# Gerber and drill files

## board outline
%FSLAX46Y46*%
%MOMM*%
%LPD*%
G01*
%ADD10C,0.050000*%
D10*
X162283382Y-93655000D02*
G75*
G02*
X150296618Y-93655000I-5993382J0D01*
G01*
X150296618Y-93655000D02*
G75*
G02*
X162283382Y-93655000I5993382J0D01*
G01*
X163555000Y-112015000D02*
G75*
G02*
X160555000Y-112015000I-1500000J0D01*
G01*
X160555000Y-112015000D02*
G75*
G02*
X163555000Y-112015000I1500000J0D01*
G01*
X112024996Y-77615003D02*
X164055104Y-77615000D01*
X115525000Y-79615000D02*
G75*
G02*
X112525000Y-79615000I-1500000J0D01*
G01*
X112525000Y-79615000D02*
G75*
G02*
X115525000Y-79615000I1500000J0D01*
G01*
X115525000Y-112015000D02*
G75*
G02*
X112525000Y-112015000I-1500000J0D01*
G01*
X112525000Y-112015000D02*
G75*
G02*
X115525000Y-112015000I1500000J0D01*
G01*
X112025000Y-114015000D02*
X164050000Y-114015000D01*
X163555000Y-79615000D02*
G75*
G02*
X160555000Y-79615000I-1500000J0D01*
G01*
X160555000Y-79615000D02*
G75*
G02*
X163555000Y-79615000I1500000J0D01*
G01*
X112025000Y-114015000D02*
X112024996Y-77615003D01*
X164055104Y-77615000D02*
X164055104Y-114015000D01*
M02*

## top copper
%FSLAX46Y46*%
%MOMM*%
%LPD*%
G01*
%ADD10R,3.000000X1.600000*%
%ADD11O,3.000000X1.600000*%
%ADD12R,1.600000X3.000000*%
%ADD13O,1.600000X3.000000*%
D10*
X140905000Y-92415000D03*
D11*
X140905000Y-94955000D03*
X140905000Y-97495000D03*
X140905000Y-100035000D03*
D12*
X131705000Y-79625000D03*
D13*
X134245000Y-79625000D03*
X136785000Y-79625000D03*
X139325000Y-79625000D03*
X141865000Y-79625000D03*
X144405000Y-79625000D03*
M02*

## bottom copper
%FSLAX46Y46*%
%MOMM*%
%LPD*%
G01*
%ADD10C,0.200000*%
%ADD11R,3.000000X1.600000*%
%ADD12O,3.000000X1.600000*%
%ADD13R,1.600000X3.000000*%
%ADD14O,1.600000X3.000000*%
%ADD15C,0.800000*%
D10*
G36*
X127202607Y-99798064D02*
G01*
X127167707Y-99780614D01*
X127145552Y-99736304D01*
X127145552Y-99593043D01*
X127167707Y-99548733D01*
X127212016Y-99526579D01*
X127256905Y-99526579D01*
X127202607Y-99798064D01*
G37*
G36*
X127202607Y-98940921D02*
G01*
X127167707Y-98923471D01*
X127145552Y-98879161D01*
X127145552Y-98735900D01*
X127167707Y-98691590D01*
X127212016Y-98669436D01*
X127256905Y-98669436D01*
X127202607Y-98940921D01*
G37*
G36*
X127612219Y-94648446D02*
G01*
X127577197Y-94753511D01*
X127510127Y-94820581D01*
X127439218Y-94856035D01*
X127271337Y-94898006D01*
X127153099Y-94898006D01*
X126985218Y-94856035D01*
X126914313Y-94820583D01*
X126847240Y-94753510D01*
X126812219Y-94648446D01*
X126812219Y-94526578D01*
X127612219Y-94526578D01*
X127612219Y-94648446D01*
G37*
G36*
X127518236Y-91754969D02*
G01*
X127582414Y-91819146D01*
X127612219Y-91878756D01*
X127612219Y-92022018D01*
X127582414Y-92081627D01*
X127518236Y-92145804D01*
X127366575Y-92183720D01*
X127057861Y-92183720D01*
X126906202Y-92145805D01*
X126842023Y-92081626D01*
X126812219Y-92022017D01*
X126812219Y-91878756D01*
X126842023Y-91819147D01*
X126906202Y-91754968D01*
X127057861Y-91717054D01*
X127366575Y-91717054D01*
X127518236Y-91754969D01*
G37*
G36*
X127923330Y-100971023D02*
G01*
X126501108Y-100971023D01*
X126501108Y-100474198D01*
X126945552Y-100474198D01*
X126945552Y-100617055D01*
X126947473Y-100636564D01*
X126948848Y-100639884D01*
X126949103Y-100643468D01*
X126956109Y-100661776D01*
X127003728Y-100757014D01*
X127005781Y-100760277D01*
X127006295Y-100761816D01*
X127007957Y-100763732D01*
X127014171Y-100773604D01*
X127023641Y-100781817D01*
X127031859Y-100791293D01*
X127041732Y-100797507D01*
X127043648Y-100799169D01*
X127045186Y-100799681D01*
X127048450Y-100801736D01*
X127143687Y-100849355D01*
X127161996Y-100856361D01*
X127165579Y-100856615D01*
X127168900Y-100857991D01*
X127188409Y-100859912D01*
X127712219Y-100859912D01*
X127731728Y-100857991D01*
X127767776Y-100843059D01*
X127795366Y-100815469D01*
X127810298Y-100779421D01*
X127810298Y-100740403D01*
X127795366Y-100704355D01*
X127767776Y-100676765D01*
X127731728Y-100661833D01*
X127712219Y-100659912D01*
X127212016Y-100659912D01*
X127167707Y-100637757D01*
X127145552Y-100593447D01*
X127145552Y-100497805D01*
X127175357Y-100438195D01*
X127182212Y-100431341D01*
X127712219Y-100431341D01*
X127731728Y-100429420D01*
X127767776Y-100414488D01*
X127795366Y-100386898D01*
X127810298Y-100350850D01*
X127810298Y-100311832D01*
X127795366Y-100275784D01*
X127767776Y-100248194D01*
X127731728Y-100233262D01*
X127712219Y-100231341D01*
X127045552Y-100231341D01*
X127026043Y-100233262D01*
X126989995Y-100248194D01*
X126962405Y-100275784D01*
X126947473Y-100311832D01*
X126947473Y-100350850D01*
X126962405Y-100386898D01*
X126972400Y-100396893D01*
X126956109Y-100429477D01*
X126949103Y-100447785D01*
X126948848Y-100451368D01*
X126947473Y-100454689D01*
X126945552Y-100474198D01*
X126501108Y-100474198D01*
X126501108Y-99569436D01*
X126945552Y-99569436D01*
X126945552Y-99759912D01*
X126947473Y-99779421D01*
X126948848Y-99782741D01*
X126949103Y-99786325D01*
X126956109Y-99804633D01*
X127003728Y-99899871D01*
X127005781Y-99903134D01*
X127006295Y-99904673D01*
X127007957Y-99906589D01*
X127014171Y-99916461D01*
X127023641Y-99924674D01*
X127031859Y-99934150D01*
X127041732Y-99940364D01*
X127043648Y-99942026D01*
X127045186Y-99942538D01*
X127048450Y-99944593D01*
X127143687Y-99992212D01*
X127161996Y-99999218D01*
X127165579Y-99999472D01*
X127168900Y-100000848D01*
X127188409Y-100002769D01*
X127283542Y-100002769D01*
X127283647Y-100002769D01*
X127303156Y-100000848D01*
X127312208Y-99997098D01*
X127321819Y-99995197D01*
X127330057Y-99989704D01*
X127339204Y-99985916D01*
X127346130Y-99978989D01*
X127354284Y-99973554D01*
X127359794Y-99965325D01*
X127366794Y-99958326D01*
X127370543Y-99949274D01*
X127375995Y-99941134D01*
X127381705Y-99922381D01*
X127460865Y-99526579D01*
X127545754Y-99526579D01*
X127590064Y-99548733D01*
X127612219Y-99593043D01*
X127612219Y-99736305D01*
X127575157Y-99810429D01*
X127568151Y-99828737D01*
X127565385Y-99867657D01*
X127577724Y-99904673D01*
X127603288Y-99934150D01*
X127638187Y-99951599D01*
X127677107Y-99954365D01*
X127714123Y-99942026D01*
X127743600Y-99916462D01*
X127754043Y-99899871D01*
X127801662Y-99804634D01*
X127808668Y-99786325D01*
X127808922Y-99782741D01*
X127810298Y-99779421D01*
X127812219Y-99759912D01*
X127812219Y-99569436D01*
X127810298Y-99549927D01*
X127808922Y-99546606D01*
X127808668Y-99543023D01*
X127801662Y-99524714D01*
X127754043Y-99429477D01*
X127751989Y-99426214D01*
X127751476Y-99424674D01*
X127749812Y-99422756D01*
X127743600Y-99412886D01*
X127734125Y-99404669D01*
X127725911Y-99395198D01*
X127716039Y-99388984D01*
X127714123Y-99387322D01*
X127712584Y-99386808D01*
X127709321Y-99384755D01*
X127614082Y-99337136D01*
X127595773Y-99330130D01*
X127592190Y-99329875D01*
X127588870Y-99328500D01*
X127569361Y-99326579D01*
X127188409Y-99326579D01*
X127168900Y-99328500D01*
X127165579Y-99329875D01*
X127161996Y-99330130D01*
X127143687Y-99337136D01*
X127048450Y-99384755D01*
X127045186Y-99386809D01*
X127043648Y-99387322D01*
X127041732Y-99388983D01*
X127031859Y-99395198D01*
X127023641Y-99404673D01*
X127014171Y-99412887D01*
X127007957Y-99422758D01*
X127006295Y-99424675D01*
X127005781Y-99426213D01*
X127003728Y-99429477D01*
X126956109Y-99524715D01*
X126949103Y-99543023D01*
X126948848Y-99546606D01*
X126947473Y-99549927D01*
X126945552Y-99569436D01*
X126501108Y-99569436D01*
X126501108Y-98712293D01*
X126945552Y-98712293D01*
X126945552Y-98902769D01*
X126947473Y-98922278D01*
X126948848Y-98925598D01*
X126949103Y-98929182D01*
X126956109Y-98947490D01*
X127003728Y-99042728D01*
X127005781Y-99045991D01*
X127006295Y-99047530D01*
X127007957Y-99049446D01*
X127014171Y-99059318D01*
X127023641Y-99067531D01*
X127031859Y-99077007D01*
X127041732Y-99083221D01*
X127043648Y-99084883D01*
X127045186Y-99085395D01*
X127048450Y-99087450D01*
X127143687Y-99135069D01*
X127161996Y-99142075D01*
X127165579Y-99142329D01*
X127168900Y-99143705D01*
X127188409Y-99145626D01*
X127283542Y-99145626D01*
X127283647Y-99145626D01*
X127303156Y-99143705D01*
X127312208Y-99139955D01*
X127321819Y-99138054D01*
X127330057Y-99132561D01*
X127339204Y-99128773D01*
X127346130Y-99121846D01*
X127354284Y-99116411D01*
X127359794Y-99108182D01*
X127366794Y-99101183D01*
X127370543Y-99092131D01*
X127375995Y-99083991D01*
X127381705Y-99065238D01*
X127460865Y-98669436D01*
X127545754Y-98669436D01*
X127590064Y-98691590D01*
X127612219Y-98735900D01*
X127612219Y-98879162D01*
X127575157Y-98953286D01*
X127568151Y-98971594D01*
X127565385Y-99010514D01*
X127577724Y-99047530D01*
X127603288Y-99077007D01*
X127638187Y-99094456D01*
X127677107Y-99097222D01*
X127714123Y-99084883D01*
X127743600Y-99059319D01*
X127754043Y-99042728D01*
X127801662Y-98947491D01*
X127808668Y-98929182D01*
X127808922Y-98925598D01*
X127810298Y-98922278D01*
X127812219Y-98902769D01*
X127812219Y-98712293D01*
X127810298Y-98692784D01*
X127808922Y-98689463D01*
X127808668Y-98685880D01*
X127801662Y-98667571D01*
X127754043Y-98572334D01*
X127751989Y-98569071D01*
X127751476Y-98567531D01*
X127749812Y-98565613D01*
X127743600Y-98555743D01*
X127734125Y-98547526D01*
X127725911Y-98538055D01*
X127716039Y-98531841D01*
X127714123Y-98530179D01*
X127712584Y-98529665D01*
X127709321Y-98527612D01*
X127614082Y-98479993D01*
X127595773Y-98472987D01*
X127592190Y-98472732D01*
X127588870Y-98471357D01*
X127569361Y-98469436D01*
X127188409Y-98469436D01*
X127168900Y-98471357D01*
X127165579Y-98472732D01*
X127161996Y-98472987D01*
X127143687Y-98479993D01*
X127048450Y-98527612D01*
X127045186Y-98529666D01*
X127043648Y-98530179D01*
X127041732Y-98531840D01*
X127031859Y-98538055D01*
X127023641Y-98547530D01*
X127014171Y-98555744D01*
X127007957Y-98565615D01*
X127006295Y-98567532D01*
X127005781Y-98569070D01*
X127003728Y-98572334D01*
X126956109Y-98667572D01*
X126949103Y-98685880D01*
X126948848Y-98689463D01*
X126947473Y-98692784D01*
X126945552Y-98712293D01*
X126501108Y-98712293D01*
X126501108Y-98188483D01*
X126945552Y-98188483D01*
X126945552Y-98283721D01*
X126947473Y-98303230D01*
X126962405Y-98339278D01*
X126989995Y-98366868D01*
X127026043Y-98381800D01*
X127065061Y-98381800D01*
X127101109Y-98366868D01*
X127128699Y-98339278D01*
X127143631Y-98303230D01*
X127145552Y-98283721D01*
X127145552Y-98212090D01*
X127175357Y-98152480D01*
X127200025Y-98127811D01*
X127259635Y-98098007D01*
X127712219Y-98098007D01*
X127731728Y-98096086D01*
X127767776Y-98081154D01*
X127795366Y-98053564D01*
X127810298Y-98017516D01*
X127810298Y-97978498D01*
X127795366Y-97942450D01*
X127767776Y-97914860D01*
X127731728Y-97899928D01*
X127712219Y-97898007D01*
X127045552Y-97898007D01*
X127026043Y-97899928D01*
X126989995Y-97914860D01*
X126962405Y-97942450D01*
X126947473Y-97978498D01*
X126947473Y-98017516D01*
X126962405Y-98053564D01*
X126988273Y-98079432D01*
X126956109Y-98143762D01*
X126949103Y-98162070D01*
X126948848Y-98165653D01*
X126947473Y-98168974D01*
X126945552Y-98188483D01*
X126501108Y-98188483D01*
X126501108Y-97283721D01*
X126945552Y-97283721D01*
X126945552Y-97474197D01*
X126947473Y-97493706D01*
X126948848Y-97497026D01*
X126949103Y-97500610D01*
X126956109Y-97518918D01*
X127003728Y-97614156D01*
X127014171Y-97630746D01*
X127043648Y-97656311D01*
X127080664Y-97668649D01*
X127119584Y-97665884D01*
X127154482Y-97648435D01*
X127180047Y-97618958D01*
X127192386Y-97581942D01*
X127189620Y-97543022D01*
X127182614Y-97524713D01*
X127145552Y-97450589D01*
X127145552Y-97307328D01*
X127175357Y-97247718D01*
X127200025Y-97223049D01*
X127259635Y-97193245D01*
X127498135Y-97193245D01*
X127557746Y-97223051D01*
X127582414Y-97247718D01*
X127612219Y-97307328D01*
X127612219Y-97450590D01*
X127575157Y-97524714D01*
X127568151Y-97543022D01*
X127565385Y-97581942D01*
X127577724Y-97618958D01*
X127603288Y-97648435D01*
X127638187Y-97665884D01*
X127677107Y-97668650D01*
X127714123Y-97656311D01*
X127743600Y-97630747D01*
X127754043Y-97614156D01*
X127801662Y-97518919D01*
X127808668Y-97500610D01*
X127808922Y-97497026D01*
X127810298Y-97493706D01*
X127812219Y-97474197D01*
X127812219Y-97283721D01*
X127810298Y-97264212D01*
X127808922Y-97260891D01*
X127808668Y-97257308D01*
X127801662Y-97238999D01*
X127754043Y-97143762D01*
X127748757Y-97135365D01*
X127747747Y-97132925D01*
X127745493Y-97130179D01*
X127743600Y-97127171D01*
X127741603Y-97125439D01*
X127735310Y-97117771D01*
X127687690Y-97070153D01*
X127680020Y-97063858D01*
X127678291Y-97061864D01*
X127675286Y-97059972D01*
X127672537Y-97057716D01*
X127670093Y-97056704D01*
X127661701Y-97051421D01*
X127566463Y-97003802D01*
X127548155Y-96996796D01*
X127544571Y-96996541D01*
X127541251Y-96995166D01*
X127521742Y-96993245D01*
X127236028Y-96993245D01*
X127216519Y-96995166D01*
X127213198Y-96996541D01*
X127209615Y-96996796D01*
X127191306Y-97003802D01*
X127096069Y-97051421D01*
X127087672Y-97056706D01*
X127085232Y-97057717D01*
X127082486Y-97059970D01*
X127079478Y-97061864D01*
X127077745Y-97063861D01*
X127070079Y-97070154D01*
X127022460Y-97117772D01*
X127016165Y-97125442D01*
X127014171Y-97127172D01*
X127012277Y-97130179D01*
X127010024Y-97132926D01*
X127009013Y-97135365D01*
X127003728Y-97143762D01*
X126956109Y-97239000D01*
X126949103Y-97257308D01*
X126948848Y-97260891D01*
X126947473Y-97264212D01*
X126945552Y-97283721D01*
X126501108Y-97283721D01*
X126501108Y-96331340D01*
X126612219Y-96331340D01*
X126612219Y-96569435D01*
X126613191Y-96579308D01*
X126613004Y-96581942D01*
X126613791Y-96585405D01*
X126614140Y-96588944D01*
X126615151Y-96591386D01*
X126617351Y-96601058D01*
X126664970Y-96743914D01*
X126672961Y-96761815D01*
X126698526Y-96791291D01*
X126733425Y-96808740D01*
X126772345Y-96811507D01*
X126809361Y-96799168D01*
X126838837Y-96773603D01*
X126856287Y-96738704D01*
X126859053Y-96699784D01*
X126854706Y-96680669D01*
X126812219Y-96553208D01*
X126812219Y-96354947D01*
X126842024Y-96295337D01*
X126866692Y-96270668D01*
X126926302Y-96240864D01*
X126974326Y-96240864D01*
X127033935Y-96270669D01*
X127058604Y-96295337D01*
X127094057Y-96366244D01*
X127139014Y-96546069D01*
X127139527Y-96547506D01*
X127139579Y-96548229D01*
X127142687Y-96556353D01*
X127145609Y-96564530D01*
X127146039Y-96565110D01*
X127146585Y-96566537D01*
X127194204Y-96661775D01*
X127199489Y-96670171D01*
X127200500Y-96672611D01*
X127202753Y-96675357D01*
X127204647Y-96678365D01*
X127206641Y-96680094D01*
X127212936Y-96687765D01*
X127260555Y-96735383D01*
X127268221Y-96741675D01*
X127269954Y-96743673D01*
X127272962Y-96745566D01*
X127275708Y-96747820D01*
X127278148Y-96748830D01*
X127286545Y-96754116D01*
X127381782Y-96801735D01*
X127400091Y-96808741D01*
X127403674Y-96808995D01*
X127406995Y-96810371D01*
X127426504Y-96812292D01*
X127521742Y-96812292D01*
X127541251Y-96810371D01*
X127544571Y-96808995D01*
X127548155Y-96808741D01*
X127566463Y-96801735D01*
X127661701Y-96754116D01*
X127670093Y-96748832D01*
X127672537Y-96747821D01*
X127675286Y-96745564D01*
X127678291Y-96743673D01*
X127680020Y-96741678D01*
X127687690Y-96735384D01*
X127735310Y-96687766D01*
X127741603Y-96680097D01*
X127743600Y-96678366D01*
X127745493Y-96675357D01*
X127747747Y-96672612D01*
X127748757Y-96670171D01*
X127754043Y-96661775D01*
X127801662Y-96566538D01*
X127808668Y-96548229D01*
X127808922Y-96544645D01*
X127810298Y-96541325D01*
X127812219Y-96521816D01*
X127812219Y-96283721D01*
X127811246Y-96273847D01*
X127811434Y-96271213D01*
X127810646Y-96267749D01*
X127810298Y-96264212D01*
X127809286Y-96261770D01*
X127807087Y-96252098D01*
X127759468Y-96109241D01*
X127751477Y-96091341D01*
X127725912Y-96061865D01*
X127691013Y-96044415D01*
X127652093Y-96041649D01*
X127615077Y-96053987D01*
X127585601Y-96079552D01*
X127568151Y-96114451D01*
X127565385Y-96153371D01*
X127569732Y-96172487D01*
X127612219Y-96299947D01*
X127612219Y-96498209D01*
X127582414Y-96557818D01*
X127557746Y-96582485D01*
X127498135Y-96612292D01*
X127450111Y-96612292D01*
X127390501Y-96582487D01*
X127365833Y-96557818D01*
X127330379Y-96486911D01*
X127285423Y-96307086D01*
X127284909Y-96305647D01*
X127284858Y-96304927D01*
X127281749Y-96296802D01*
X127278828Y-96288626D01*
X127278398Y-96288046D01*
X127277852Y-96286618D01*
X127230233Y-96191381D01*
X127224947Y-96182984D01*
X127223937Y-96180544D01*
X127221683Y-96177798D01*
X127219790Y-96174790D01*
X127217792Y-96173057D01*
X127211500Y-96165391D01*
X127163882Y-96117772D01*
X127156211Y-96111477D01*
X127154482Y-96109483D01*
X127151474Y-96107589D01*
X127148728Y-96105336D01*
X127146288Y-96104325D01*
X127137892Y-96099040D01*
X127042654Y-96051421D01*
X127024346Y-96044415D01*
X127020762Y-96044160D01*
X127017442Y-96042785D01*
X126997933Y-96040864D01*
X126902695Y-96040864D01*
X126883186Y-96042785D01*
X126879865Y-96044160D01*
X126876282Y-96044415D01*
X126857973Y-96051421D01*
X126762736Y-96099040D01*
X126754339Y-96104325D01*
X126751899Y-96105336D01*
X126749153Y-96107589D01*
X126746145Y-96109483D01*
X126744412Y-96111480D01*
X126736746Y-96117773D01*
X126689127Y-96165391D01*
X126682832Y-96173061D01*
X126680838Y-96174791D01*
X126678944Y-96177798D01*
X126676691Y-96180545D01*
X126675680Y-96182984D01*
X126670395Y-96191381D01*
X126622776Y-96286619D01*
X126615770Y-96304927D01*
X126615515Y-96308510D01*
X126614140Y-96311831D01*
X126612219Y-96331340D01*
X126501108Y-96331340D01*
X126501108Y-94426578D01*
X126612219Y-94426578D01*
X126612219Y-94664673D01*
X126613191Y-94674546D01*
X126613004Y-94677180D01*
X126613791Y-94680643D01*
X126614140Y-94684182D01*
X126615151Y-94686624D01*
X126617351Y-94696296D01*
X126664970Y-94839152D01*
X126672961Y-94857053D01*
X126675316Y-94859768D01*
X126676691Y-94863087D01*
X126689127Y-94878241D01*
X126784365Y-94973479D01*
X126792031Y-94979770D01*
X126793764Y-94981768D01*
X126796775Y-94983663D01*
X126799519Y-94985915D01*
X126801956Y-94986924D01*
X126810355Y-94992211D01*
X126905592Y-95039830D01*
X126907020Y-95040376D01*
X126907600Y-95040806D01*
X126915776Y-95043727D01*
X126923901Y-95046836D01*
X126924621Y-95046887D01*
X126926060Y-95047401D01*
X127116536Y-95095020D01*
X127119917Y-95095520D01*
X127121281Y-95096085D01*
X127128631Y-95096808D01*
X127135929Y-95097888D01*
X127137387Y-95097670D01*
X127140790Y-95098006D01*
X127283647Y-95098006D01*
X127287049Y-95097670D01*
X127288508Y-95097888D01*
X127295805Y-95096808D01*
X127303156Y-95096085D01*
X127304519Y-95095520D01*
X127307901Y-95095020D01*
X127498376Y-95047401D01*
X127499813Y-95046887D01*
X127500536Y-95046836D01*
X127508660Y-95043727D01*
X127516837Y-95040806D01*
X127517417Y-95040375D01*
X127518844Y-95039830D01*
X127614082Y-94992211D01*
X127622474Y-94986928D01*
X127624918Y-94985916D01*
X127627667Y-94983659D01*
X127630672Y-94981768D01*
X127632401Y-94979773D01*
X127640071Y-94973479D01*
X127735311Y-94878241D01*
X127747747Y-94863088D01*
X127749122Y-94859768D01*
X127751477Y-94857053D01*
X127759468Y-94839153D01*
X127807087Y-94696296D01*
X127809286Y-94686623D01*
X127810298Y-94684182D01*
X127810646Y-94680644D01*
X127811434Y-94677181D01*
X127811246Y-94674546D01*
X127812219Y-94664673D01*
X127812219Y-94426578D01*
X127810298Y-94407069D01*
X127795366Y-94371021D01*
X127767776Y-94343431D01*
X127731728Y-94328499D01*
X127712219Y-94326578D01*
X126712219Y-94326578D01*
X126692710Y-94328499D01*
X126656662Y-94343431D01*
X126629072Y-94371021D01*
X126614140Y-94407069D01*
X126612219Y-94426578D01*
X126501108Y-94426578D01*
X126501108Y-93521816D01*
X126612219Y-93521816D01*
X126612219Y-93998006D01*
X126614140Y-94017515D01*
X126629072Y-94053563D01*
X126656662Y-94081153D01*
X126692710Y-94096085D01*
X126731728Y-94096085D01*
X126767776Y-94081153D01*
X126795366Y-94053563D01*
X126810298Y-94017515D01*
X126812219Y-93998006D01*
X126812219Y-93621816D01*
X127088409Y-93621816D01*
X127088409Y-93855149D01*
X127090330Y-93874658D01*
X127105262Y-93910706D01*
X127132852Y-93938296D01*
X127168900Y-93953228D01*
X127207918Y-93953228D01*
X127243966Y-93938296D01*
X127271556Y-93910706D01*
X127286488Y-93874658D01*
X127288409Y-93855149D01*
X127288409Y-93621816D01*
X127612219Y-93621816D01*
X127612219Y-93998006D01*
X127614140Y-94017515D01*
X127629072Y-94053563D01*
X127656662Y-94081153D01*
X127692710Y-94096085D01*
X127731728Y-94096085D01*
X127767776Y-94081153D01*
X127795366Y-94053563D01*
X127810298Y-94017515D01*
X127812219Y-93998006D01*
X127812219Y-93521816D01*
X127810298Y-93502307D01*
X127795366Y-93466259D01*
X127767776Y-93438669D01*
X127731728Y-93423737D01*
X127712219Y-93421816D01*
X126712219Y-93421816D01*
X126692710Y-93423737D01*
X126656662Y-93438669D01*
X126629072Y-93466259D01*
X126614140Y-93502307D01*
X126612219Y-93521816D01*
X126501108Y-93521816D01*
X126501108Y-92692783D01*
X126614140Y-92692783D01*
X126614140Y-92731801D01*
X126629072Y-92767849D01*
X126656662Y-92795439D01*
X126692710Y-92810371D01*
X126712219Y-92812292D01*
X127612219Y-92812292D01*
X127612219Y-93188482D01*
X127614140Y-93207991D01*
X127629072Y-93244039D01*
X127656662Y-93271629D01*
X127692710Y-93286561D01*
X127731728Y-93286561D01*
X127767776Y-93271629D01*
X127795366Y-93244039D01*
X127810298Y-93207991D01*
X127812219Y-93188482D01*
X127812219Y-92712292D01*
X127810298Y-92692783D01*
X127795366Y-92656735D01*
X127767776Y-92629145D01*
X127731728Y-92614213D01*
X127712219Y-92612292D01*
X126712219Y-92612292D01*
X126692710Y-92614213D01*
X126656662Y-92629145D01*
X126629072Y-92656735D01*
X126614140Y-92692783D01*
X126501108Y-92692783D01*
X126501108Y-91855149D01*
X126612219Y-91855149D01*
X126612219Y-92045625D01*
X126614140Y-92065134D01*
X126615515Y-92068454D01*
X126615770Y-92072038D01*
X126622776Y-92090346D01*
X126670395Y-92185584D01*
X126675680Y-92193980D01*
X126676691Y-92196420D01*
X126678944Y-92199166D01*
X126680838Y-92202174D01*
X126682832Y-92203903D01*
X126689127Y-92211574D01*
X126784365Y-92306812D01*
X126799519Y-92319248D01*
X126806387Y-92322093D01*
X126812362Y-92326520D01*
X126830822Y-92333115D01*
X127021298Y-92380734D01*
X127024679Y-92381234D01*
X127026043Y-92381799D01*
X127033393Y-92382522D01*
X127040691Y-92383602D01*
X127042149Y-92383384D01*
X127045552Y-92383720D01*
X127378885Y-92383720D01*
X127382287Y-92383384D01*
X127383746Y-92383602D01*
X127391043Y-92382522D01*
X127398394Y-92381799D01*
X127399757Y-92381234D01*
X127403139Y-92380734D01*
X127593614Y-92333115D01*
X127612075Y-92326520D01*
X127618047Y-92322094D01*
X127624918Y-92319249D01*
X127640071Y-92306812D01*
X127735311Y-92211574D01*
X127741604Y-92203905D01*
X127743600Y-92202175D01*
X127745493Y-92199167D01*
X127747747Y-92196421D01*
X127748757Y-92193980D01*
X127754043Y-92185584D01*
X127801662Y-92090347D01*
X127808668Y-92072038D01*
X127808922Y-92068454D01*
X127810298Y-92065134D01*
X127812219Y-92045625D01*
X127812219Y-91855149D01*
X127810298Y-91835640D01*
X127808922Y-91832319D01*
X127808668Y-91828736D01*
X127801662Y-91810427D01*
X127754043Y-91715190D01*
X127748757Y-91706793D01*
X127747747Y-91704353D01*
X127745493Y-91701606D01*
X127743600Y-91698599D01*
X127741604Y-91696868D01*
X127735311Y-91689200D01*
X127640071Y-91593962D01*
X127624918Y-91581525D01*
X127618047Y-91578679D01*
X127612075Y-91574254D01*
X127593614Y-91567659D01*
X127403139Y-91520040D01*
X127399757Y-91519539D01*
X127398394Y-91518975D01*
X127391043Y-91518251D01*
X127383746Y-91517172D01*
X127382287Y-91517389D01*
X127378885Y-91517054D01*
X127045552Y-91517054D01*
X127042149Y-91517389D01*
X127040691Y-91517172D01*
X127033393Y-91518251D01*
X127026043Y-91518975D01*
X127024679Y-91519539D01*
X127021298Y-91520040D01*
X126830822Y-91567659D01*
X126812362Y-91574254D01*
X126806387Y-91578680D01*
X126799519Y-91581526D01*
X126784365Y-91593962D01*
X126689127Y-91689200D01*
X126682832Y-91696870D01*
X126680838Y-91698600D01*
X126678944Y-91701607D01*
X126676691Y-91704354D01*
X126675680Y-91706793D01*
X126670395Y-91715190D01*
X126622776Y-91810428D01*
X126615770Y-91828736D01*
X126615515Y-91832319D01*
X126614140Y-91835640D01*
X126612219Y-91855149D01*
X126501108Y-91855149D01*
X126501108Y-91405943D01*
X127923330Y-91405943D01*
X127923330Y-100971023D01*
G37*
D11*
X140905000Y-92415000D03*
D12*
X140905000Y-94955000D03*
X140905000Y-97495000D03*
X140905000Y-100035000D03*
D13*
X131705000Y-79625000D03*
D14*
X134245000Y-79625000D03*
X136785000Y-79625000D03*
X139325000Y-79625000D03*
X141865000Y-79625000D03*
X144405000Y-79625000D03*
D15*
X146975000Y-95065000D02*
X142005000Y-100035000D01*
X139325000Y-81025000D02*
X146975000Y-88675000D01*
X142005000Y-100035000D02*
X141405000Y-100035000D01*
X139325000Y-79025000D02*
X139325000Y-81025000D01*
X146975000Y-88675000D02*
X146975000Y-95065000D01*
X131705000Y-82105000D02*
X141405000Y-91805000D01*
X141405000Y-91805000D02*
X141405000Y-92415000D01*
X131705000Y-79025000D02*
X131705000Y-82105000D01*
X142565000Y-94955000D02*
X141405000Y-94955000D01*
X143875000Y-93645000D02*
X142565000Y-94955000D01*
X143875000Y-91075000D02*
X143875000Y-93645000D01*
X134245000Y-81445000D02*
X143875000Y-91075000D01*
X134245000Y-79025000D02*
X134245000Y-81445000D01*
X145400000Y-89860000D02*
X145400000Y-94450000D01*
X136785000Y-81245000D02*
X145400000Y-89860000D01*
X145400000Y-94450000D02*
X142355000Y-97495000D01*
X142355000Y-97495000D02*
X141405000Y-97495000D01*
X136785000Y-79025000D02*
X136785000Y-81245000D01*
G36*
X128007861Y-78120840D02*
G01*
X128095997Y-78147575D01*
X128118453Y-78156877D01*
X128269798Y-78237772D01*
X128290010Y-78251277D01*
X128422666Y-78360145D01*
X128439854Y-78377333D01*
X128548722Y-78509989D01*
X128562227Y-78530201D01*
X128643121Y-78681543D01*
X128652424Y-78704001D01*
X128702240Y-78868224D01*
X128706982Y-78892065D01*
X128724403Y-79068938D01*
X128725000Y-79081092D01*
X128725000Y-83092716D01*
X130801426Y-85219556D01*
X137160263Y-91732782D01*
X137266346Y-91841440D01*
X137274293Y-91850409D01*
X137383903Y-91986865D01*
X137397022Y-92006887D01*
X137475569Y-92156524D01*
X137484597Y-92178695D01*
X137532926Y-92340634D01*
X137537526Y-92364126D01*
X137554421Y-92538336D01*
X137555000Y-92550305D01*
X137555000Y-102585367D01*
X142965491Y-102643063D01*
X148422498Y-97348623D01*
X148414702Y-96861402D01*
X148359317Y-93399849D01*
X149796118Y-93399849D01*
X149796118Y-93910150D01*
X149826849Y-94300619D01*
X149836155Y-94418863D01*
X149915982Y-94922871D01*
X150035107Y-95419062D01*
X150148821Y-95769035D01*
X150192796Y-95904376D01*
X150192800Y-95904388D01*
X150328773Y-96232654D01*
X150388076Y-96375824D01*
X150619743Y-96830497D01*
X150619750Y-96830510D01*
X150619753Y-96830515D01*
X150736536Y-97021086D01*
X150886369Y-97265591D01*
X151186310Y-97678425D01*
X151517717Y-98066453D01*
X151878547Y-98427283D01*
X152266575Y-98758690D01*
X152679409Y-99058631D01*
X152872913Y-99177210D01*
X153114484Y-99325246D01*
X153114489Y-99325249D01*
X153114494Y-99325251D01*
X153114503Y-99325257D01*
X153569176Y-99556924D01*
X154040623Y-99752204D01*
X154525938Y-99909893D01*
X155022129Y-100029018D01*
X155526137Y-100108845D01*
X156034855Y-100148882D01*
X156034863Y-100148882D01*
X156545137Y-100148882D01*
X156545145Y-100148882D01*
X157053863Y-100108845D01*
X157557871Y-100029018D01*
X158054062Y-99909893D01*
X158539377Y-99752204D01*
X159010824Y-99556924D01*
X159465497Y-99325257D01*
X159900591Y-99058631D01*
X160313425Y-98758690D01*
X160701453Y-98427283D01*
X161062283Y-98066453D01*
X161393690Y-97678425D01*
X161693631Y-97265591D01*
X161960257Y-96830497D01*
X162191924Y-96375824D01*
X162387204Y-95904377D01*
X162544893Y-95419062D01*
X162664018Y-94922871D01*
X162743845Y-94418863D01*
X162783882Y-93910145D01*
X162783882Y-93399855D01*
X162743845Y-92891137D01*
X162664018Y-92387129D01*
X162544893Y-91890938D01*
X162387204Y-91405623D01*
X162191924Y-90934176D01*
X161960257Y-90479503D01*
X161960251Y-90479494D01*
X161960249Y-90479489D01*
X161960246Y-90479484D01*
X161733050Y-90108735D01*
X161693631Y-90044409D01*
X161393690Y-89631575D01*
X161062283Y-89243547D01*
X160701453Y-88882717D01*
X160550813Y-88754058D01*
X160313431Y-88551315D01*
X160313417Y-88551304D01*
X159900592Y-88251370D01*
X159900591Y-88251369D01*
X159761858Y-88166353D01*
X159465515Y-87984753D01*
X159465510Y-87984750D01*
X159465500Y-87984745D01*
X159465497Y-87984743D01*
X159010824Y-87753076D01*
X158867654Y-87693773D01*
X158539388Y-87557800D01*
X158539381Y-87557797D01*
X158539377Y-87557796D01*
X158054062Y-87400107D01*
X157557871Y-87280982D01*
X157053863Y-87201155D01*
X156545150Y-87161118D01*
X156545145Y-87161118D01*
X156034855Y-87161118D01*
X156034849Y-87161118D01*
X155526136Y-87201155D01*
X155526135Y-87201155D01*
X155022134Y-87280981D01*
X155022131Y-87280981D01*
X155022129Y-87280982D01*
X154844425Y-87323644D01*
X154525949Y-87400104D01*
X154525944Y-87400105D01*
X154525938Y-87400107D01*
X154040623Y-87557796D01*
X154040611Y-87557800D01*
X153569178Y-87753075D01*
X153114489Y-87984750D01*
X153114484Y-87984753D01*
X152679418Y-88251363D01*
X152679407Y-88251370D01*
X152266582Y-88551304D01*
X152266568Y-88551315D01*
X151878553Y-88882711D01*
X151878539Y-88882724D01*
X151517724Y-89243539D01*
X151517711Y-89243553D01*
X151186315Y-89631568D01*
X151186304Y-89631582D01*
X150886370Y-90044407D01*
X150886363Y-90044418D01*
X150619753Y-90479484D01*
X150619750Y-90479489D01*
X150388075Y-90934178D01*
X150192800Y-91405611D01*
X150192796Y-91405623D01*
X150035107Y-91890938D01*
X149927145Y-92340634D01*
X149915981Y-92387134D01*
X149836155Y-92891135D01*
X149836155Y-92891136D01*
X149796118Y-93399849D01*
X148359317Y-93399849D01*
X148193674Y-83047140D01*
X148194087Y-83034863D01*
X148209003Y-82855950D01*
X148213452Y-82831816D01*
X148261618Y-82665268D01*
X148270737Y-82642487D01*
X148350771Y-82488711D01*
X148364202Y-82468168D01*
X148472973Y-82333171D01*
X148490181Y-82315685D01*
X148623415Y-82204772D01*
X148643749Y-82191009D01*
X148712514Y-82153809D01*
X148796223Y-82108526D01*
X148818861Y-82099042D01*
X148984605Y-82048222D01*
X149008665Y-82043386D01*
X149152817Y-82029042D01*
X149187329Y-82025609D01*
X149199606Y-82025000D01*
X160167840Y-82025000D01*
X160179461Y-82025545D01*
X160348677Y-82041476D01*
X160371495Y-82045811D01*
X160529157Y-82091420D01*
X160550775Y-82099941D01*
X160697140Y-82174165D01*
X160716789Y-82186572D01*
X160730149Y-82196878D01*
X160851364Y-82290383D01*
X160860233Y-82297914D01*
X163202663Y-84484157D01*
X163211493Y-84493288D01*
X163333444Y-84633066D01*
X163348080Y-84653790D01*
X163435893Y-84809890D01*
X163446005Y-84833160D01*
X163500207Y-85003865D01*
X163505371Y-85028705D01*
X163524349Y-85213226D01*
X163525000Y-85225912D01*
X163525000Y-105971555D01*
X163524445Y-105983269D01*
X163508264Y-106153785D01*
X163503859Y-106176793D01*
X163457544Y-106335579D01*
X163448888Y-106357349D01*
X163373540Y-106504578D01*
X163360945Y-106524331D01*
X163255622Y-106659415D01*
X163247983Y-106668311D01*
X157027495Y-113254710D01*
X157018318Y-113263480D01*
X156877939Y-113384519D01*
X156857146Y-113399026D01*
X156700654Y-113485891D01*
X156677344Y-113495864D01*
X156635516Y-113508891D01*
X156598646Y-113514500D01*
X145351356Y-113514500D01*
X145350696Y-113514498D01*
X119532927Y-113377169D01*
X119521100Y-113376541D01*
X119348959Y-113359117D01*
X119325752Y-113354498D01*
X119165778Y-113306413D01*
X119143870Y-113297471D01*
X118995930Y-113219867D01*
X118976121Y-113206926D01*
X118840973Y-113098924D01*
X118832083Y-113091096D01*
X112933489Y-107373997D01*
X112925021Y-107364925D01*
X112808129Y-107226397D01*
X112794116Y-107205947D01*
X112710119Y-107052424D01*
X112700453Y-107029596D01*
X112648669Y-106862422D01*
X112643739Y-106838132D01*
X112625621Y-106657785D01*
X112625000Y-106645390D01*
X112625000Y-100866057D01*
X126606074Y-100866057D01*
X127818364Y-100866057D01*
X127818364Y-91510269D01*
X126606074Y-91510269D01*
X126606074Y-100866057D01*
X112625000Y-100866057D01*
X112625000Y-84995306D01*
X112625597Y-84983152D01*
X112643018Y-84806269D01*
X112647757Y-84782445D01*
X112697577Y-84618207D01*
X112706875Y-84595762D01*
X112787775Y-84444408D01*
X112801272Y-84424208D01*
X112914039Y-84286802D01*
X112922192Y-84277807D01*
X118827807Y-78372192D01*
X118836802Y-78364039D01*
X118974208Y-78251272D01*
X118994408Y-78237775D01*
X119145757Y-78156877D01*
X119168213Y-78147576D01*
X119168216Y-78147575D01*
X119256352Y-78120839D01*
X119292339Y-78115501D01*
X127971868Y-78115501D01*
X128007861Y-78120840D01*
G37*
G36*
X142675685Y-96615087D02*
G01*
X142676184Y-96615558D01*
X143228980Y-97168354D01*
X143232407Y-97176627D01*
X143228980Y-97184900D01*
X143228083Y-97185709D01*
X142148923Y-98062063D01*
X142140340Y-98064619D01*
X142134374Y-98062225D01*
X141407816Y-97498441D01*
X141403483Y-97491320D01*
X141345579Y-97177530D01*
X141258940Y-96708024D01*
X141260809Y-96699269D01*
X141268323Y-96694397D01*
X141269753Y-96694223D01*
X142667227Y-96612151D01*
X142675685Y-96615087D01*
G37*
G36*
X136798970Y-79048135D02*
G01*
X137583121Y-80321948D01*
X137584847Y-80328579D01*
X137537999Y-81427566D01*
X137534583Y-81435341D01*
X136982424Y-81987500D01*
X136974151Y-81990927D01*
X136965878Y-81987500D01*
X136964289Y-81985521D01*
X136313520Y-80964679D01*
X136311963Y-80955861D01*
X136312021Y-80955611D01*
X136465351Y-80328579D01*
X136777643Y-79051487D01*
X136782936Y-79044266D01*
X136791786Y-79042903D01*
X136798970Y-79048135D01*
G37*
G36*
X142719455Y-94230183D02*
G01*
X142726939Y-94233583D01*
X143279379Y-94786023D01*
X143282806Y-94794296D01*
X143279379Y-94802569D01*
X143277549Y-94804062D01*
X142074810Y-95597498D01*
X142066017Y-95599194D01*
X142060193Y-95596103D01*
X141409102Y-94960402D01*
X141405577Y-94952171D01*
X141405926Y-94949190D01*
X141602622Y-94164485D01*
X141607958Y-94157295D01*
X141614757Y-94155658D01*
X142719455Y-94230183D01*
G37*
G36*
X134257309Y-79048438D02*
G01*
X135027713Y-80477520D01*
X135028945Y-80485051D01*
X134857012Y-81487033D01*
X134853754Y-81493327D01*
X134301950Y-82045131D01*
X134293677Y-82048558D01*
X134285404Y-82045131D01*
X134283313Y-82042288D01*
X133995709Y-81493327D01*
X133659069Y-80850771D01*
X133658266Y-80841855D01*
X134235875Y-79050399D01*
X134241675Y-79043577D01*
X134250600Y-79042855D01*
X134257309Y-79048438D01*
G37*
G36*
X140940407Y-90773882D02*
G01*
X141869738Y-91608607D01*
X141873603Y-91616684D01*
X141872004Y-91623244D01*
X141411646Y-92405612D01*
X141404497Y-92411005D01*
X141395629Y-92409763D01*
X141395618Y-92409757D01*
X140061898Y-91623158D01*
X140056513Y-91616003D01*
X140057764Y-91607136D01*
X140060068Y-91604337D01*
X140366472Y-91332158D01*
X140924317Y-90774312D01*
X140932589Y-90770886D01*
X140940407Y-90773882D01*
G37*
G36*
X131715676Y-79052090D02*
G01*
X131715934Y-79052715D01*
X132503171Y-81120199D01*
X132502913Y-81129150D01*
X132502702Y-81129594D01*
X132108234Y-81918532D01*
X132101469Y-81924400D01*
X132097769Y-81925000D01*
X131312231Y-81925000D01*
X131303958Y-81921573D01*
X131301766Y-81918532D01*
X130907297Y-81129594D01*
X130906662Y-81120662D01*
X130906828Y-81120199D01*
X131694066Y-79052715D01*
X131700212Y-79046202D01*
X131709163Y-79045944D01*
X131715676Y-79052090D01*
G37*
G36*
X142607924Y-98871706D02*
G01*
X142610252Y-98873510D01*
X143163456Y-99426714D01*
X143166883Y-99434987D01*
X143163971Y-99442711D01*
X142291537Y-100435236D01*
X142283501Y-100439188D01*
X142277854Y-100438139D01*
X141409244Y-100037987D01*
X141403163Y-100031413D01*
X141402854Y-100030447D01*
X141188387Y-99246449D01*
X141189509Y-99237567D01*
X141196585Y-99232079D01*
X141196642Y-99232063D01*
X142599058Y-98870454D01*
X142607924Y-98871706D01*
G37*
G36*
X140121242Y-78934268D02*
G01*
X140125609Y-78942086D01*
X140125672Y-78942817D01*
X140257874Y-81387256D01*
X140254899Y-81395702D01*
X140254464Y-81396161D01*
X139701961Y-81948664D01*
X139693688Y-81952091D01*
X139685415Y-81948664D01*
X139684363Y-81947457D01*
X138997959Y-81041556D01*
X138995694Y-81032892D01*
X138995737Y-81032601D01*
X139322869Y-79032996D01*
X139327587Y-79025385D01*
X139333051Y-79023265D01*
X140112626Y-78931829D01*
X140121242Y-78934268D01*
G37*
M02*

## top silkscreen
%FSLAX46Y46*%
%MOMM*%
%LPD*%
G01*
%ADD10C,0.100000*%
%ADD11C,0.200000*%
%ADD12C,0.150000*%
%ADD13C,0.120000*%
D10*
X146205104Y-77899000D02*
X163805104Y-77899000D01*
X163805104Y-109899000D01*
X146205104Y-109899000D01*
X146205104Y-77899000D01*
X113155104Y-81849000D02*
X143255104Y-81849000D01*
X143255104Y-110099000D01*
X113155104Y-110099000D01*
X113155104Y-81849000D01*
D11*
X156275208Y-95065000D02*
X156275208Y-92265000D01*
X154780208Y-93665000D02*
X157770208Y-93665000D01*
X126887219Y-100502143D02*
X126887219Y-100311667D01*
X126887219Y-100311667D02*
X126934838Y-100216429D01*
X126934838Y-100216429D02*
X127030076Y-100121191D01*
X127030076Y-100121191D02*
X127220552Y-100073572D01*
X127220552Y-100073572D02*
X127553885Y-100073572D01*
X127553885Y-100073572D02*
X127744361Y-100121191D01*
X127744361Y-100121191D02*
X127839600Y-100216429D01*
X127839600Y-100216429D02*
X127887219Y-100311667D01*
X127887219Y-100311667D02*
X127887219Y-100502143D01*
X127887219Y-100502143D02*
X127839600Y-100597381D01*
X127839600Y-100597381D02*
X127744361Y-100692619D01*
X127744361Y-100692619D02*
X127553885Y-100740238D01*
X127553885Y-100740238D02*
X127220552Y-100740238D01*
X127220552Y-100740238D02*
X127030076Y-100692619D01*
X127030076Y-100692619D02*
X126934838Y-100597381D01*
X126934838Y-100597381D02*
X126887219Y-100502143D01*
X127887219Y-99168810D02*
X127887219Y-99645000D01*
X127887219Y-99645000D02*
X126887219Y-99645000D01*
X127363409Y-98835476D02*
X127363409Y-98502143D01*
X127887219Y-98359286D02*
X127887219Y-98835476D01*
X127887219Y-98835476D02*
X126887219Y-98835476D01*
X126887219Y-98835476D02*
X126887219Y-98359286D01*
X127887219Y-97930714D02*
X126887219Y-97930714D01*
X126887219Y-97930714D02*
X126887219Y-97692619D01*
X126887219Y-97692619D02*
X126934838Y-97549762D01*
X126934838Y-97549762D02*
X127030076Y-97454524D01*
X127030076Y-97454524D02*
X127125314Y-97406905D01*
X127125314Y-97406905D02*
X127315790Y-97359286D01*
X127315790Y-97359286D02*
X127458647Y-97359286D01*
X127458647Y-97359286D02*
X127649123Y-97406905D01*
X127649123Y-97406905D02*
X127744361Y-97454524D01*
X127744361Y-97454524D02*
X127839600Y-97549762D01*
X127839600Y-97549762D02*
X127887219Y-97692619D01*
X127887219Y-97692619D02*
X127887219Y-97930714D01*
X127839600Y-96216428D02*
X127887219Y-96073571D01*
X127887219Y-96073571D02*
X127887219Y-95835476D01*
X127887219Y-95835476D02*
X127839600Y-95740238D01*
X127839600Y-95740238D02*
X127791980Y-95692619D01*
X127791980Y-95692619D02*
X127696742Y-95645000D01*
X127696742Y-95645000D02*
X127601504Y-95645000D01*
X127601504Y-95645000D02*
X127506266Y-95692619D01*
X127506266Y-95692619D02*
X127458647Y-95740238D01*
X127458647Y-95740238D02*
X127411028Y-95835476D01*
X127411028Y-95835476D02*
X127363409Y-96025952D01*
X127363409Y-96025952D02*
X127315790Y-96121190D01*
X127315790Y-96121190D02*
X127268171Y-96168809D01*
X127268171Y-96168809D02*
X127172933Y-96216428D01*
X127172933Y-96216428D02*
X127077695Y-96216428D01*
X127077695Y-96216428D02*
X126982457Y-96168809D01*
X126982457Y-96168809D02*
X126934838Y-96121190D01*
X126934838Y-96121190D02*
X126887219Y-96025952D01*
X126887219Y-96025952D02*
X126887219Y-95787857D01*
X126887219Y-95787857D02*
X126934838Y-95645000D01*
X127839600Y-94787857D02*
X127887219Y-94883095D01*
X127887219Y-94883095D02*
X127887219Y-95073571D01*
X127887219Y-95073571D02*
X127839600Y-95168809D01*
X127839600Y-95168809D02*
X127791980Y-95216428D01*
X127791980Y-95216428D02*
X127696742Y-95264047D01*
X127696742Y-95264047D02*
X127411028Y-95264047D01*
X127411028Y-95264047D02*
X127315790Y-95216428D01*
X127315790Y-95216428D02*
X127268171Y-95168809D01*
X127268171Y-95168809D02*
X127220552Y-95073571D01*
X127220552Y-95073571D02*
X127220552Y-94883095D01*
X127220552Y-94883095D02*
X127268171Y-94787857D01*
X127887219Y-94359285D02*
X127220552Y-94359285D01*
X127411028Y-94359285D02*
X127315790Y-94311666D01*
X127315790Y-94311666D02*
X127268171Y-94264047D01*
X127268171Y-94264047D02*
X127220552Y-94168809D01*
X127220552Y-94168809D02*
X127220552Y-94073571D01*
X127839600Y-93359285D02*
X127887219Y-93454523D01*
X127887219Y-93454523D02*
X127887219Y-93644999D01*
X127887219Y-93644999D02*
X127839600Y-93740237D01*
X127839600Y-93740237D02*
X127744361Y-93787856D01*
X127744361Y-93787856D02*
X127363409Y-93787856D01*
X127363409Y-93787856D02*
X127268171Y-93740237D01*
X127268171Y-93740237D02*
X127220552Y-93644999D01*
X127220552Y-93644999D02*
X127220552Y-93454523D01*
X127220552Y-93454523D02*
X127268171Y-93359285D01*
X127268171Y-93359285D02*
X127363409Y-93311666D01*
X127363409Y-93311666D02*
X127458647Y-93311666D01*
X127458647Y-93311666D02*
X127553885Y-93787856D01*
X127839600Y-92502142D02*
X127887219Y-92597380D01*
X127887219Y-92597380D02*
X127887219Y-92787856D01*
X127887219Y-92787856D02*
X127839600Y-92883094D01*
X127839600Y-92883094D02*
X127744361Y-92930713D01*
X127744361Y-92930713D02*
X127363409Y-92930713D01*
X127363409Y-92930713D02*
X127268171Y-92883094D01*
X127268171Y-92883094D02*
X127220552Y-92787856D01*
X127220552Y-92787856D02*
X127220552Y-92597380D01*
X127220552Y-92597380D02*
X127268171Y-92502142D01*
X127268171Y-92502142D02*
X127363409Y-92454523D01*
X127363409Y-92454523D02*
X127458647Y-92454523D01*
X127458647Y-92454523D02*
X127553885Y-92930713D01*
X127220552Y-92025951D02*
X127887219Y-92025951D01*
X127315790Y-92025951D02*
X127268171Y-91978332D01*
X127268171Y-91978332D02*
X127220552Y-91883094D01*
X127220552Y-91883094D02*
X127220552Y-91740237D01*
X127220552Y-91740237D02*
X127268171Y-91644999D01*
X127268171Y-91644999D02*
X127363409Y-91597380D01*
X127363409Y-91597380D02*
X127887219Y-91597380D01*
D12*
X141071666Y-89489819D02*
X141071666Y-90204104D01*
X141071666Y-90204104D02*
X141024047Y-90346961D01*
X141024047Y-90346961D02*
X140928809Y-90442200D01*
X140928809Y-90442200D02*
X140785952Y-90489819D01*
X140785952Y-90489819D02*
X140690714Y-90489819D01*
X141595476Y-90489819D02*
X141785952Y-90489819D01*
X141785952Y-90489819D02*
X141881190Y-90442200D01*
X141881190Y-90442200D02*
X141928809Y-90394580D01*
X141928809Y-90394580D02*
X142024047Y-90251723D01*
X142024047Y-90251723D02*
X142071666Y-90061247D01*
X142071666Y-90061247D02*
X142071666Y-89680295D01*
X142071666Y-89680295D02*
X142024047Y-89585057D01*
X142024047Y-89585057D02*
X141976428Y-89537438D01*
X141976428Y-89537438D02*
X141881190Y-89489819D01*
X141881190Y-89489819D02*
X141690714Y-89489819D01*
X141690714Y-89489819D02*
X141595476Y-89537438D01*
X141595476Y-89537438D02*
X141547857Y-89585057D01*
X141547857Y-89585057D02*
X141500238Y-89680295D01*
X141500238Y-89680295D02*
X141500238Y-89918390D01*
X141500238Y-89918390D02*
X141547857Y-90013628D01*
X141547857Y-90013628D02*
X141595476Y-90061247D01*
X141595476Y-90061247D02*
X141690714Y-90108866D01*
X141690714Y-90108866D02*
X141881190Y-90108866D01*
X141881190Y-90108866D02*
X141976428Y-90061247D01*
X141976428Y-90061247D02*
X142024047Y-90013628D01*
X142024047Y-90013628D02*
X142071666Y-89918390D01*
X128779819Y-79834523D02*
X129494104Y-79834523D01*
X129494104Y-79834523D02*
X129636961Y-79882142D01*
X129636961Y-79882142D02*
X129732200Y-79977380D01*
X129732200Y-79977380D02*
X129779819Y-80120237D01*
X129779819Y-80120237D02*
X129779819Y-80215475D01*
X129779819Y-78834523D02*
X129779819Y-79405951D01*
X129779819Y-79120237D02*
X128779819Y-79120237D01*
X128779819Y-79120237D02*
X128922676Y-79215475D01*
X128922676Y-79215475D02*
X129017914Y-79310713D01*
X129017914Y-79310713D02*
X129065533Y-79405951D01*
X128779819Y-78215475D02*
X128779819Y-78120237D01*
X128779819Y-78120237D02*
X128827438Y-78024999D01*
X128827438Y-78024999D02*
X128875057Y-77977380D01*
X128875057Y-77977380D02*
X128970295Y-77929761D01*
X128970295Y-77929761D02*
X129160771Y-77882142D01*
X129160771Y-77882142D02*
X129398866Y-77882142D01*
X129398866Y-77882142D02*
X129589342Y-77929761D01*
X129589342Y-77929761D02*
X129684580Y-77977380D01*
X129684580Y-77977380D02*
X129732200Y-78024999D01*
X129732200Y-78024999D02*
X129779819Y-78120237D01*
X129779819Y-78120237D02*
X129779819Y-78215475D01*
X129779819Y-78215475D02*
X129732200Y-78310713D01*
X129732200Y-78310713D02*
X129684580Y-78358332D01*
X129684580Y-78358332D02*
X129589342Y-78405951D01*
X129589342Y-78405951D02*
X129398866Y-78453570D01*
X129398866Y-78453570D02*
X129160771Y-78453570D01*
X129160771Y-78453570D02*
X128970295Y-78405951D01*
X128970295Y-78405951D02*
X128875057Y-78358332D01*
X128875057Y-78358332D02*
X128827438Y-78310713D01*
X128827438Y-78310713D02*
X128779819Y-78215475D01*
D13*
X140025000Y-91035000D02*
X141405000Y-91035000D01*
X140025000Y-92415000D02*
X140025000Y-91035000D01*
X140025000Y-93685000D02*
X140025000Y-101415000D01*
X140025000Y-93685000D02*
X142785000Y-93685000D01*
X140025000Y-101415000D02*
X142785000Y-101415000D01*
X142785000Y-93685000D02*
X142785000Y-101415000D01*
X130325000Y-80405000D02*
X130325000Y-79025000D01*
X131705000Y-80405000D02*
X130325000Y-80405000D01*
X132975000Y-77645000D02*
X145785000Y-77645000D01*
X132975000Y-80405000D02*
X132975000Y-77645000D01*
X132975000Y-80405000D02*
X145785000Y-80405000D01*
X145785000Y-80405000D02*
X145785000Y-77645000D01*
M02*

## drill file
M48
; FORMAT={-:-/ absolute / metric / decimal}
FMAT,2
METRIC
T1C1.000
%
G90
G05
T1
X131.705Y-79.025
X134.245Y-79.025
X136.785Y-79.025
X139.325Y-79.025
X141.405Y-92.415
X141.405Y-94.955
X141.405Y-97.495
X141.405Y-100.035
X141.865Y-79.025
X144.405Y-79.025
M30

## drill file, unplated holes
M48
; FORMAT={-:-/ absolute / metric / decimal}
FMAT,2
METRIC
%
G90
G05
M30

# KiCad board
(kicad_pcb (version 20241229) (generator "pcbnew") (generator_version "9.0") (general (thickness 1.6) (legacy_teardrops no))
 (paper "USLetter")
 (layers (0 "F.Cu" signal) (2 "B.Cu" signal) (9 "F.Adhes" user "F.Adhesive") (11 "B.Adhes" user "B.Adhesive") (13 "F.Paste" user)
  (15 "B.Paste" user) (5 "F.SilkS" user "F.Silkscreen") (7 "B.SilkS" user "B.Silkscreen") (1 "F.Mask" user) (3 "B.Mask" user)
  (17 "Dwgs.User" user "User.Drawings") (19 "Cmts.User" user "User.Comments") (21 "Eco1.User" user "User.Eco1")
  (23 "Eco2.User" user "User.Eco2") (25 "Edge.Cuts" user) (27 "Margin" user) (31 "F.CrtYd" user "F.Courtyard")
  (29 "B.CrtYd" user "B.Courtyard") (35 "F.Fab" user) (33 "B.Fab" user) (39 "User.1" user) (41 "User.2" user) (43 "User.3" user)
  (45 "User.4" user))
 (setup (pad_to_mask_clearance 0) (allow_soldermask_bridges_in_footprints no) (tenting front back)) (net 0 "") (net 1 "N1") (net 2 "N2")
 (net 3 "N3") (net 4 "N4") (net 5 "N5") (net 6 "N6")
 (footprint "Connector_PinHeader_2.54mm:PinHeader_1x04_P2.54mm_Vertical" (layer "F.Cu") (at 141.405 92.415)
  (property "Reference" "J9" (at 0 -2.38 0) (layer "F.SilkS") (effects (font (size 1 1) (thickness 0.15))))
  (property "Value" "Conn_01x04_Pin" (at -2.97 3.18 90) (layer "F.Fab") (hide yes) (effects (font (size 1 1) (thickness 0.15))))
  (fp_line (start -1.38 -1.38) (end 0 -1.38) (stroke (width 0.12) (type solid)) (layer "F.SilkS"))
  (fp_line (start -1.38 0) (end -1.38 -1.38) (stroke (width 0.12) (type solid)) (layer "F.SilkS"))
  (fp_line (start -1.38 1.27) (end -1.38 9) (stroke (width 0.12) (type solid)) (layer "F.SilkS"))
  (fp_line (start -1.38 1.27) (end 1.38 1.27) (stroke (width 0.12) (type solid)) (layer "F.SilkS"))
  (fp_line (start -1.38 9) (end 1.38 9) (stroke (width 0.12) (type solid)) (layer "F.SilkS"))
  (fp_line (start 1.38 1.27) (end 1.38 9) (stroke (width 0.12) (type solid)) (layer "F.SilkS"))
  (pad "1" thru_hole rect (at 0 0) (size 3 1.6) (drill 1 (offset -0.5 0)) (layers "*.Cu" "*.Mask") (remove_unused_layers no) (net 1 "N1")
   (teardrops (best_length_ratio 0.5) (max_length 1) (best_width_ratio 1) (max_width 2) (curved_edges no) (filter_ratio 0.9) (enabled yes)
    (allow_two_segments yes) (prefer_zone_connections yes)))
  (pad "2" thru_hole oval (at 0 2.54) (size 3 1.6) (drill 1 (offset -0.5 0)) (layers "*.Cu" "*.Mask" "B.Paste") (remove_unused_layers no)
   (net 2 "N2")
   (teardrops (best_length_ratio 0.5) (max_length 1) (best_width_ratio 1) (max_width 2) (curved_edges no) (filter_ratio 0.9) (enabled yes)
    (allow_two_segments yes) (prefer_zone_connections yes)))
  (pad "3" thru_hole oval (at 0 5.08) (size 3 1.6) (drill 1 (offset -0.5 0)) (layers "*.Cu" "*.Mask" "B.Paste") (remove_unused_layers no)
   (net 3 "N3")
   (teardrops (best_length_ratio 0.5) (max_length 1) (best_width_ratio 1) (max_width 2) (curved_edges no) (filter_ratio 0.9) (enabled yes)
    (allow_two_segments yes) (prefer_zone_connections yes)))
  (pad "4" thru_hole oval (at 0 7.62) (size 3 1.6) (drill 1 (offset -0.5 0)) (layers "*.Cu" "*.Mask" "B.Paste") (remove_unused_layers no)
   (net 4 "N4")
   (teardrops (best_length_ratio 0.5) (max_length 1) (best_width_ratio 1) (max_width 2) (curved_edges no) (filter_ratio 0.9) (enabled yes)
    (allow_two_segments yes) (prefer_zone_connections yes))))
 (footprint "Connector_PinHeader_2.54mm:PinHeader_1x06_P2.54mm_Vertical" (layer "F.Cu") (at 131.705 79.025 90)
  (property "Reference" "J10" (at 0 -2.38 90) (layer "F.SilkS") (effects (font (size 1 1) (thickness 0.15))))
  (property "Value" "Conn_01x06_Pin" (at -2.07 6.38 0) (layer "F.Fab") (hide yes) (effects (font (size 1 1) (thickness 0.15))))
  (fp_line (start -1.38 -1.38) (end 0 -1.38) (stroke (width 0.12) (type solid)) (layer "F.SilkS"))
  (fp_line (start -1.38 0) (end -1.38 -1.38) (stroke (width 0.12) (type solid)) (layer "F.SilkS"))
  (fp_line (start 1.38 1.27) (end 1.38 14.08) (stroke (width 0.12) (type solid)) (layer "F.SilkS"))
  (fp_line (start -1.38 1.27) (end 1.38 1.27) (stroke (width 0.12) (type solid)) (layer "F.SilkS"))
  (fp_line (start -1.38 1.27) (end -1.38 14.08) (stroke (width 0.12) (type solid)) (layer "F.SilkS"))
  (fp_line (start -1.38 14.08) (end 1.38 14.08) (stroke (width 0.12) (type solid)) (layer "F.SilkS"))
  (pad "1" thru_hole rect (at 0 0 90) (size 3 1.6) (drill 1 (offset -0.6 0)) (layers "*.Cu" "*.Mask") (remove_unused_layers no) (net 1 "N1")
   (teardrops (best_length_ratio 0.5) (max_length 1) (best_width_ratio 1) (max_width 2) (curved_edges no) (filter_ratio 0.9) (enabled yes)
    (allow_two_segments yes) (prefer_zone_connections yes)))
  (pad "2" thru_hole oval (at 0 2.54 90) (size 3 1.6) (drill 1 (offset -0.6 0)) (layers "*.Cu" "*.Mask") (remove_unused_layers no)
   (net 2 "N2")
   (teardrops (best_length_ratio 0.5) (max_length 1) (best_width_ratio 1) (max_width 2) (curved_edges no) (filter_ratio 0.9) (enabled yes)
    (allow_two_segments yes) (prefer_zone_connections yes)))
  (pad "3" thru_hole oval (at 0 5.08 90) (size 3 1.6) (drill 1 (offset -0.6 0)) (layers "*.Cu" "*.Mask") (remove_unused_layers no)
   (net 3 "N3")
   (teardrops (best_length_ratio 0.5) (max_length 1) (best_width_ratio 1) (max_width 2) (curved_edges no) (filter_ratio 0.9) (enabled yes)
    (allow_two_segments yes) (prefer_zone_connections yes)))
  (pad "4" thru_hole oval (at 0 7.62 90) (size 3 1.6) (drill 1 (offset -0.6 0)) (layers "*.Cu" "*.Mask") (remove_unused_layers no)
   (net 4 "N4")
   (teardrops (best_length_ratio 0.5) (max_length 1) (best_width_ratio 1) (max_width 2) (curved_edges no) (filter_ratio 0.9) (enabled yes)
    (allow_two_segments yes) (prefer_zone_connections yes)))
  (pad "5" thru_hole oval (at 0 10.16 90) (size 3 1.6) (drill 1 (offset -0.6 0)) (layers "*.Cu" "*.Mask") (remove_unused_layers no)
   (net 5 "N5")
   (teardrops (best_length_ratio 0.5) (max_length 1) (best_width_ratio 1) (max_width 2) (curved_edges no) (filter_ratio 0.9) (enabled yes)
    (allow_two_segments yes) (prefer_zone_connections yes)))
  (pad "6" thru_hole oval (at 0 12.7 90) (size 3 1.6) (drill 1 (offset -0.6 0)) (layers "*.Cu" "*.Mask") (remove_unused_layers no)
   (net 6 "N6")
   (teardrops (best_length_ratio 0.5) (max_length 1) (best_width_ratio 1) (max_width 2) (curved_edges no) (filter_ratio 0.9) (enabled yes)
    (allow_two_segments yes) (prefer_zone_connections yes))))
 (gr_line (start 156.275208 95.065) (end 156.275208 92.265) (stroke (width 0.2) (type default)) (layer "F.SilkS"))
 (gr_rect (start 146.205104 77.899) (end 163.805104 109.899) (stroke (width 0.1) (type solid)) (fill no) (layer "F.SilkS"))
 (gr_line (start 154.780208 93.665) (end 157.770208 93.665) (stroke (width 0.2) (type default)) (layer "F.SilkS"))
 (gr_rect (start 113.155104 81.849) (end 143.255104 110.099) (stroke (width 0.1) (type solid)) (fill no) (layer "F.SilkS"))
 (gr_circle (center 156.29 93.655) (end 160.59 97.83) (stroke (width 0.05) (type default)) (fill no) (layer "Edge.Cuts"))
 (gr_circle (center 162.055 112.015) (end 163.555 112.015) (stroke (width 0.05) (type default)) (fill no) (layer "Edge.Cuts"))
 (gr_line (start 112.024996 77.615003) (end 164.055104 77.615) (stroke (width 0.05) (type default)) (layer "Edge.Cuts"))
 (gr_circle (center 114.025 79.615) (end 115.525 79.615) (stroke (width 0.05) (type default)) (fill no) (layer "Edge.Cuts"))
 (gr_circle (center 114.025 112.015) (end 115.525 112.015) (stroke (width 0.05) (type default)) (fill no) (layer "Edge.Cuts"))
 (gr_line (start 112.025 114.015) (end 164.05 114.015) (stroke (width 0.05) (type default)) (layer "Edge.Cuts"))
 (gr_circle (center 162.055 79.615) (end 163.555 79.615) (stroke (width 0.05) (type default)) (fill no) (layer "Edge.Cuts"))
 (gr_line (start 112.025 114.015) (end 112.024996 77.615003) (stroke (width 0.05) (type default)) (layer "Edge.Cuts"))
 (gr_line (start 164.055104 77.615) (end 164.055104 114.015) (stroke (width 0.05) (type default)) (layer "Edge.Cuts"))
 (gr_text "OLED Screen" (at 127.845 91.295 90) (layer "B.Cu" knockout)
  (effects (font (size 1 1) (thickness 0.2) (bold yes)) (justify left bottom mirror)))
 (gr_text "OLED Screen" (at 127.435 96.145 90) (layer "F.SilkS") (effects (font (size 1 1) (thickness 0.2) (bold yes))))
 (segment (start 145.4 94.45) (end 142.355 97.495) (width 0.8) (layer "B.Cu") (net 3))
 (segment (start 136.785 81.245) (end 145.4 89.86) (width 0.8) (layer "B.Cu") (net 3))
 (segment (start 136.785 79.025) (end 136.785 81.245) (width 0.8) (layer "B.Cu") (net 3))
 (segment (start 145.4 89.86) (end 145.4 94.45) (width 0.8) (layer "B.Cu") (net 3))
 (segment (start 142.355 97.495) (end 141.405 97.495) (width 0.8) (layer "B.Cu") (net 3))
 (segment (start 143.875 91.075) (end 143.875 93.645) (width 0.8) (layer "B.Cu") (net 2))
 (segment (start 134.245 79.025) (end 134.245 81.445) (width 0.8) (layer "B.Cu") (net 2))
 (segment (start 143.875 93.645) (end 142.565 94.955) (width 0.8) (layer "B.Cu") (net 2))
 (segment (start 134.245 81.445) (end 143.875 91.075) (width 0.8) (layer "B.Cu") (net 2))
 (segment (start 142.565 94.955) (end 141.405 94.955) (width 0.8) (layer "B.Cu") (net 2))
 (segment (start 146.975 95.065) (end 142.005 100.035) (width 0.8) (layer "B.Cu") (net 4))
 (segment (start 146.975 88.675) (end 146.975 95.065) (width 0.8) (layer "B.Cu") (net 4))
 (segment (start 139.325 81.025) (end 146.975 88.675) (width 0.8) (layer "B.Cu") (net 4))
 (segment (start 142.005 100.035) (end 141.405 100.035) (width 0.8) (layer "B.Cu") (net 4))
 (segment (start 139.325 79.025) (end 139.325 81.025) (width 0.8) (layer "B.Cu") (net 4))
 (segment (start 141.405 91.805) (end 141.405 92.415) (width 0.8) (layer "B.Cu") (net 1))
 (segment (start 131.705 82.105) (end 141.405 91.805) (width 0.8) (layer "B.Cu") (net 1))
 (segment (start 131.705 79.025) (end 131.705 82.105) (width 0.8) (layer "B.Cu") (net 1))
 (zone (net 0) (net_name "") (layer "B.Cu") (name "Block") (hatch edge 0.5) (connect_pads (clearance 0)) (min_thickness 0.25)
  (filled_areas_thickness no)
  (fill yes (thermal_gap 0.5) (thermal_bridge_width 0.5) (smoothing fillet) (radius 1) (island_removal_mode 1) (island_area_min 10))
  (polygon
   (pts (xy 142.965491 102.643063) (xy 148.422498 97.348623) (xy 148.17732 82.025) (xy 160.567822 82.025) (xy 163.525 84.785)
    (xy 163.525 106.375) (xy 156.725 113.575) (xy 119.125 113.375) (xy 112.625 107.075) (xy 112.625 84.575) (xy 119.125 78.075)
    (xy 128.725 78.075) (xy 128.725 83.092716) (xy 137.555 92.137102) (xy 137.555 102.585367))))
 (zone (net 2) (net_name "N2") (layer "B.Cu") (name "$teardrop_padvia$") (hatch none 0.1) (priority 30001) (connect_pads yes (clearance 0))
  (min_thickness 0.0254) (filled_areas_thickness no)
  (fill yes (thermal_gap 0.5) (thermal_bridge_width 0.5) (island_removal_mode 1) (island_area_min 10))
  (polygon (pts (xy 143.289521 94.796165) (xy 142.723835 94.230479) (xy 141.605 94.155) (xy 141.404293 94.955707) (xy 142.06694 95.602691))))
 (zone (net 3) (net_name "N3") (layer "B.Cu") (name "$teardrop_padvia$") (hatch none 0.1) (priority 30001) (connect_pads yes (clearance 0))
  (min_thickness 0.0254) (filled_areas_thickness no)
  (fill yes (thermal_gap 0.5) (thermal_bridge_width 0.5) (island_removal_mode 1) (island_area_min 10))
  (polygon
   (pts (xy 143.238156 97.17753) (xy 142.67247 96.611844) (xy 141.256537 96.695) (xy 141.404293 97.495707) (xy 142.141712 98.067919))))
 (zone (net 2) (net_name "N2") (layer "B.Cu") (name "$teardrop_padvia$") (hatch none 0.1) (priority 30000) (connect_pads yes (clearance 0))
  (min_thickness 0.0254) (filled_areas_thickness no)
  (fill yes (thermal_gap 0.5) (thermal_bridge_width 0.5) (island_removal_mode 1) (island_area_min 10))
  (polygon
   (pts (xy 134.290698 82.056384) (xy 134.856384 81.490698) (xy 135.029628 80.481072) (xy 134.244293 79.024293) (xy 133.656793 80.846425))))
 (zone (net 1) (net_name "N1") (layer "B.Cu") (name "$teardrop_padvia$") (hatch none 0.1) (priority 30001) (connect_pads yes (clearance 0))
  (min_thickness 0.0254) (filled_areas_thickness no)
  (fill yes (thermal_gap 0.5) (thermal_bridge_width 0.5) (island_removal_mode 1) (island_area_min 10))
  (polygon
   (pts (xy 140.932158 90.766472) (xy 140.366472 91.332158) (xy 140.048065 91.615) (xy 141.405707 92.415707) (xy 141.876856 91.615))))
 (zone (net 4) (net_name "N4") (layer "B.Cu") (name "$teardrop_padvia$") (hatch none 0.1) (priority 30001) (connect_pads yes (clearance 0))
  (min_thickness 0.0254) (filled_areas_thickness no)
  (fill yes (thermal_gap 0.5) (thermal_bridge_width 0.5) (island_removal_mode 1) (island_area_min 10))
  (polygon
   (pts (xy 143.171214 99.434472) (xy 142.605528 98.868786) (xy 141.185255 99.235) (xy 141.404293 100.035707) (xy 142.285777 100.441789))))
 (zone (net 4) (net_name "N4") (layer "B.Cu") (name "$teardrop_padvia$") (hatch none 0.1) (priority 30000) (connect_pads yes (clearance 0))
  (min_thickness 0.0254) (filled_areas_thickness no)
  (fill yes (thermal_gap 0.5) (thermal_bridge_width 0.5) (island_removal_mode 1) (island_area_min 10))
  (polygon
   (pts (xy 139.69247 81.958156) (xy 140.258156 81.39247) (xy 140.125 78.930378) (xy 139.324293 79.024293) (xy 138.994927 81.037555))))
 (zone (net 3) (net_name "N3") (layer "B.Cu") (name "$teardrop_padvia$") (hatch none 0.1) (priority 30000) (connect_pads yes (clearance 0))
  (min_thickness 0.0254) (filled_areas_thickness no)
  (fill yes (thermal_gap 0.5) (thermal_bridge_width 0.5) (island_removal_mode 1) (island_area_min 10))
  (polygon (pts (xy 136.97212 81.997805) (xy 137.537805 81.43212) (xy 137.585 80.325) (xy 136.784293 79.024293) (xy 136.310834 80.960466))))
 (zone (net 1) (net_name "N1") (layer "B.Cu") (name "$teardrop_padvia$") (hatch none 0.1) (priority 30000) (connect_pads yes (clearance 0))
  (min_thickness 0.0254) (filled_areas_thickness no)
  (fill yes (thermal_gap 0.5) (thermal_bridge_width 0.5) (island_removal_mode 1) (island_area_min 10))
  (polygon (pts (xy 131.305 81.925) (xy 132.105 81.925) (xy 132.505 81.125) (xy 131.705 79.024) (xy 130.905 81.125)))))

